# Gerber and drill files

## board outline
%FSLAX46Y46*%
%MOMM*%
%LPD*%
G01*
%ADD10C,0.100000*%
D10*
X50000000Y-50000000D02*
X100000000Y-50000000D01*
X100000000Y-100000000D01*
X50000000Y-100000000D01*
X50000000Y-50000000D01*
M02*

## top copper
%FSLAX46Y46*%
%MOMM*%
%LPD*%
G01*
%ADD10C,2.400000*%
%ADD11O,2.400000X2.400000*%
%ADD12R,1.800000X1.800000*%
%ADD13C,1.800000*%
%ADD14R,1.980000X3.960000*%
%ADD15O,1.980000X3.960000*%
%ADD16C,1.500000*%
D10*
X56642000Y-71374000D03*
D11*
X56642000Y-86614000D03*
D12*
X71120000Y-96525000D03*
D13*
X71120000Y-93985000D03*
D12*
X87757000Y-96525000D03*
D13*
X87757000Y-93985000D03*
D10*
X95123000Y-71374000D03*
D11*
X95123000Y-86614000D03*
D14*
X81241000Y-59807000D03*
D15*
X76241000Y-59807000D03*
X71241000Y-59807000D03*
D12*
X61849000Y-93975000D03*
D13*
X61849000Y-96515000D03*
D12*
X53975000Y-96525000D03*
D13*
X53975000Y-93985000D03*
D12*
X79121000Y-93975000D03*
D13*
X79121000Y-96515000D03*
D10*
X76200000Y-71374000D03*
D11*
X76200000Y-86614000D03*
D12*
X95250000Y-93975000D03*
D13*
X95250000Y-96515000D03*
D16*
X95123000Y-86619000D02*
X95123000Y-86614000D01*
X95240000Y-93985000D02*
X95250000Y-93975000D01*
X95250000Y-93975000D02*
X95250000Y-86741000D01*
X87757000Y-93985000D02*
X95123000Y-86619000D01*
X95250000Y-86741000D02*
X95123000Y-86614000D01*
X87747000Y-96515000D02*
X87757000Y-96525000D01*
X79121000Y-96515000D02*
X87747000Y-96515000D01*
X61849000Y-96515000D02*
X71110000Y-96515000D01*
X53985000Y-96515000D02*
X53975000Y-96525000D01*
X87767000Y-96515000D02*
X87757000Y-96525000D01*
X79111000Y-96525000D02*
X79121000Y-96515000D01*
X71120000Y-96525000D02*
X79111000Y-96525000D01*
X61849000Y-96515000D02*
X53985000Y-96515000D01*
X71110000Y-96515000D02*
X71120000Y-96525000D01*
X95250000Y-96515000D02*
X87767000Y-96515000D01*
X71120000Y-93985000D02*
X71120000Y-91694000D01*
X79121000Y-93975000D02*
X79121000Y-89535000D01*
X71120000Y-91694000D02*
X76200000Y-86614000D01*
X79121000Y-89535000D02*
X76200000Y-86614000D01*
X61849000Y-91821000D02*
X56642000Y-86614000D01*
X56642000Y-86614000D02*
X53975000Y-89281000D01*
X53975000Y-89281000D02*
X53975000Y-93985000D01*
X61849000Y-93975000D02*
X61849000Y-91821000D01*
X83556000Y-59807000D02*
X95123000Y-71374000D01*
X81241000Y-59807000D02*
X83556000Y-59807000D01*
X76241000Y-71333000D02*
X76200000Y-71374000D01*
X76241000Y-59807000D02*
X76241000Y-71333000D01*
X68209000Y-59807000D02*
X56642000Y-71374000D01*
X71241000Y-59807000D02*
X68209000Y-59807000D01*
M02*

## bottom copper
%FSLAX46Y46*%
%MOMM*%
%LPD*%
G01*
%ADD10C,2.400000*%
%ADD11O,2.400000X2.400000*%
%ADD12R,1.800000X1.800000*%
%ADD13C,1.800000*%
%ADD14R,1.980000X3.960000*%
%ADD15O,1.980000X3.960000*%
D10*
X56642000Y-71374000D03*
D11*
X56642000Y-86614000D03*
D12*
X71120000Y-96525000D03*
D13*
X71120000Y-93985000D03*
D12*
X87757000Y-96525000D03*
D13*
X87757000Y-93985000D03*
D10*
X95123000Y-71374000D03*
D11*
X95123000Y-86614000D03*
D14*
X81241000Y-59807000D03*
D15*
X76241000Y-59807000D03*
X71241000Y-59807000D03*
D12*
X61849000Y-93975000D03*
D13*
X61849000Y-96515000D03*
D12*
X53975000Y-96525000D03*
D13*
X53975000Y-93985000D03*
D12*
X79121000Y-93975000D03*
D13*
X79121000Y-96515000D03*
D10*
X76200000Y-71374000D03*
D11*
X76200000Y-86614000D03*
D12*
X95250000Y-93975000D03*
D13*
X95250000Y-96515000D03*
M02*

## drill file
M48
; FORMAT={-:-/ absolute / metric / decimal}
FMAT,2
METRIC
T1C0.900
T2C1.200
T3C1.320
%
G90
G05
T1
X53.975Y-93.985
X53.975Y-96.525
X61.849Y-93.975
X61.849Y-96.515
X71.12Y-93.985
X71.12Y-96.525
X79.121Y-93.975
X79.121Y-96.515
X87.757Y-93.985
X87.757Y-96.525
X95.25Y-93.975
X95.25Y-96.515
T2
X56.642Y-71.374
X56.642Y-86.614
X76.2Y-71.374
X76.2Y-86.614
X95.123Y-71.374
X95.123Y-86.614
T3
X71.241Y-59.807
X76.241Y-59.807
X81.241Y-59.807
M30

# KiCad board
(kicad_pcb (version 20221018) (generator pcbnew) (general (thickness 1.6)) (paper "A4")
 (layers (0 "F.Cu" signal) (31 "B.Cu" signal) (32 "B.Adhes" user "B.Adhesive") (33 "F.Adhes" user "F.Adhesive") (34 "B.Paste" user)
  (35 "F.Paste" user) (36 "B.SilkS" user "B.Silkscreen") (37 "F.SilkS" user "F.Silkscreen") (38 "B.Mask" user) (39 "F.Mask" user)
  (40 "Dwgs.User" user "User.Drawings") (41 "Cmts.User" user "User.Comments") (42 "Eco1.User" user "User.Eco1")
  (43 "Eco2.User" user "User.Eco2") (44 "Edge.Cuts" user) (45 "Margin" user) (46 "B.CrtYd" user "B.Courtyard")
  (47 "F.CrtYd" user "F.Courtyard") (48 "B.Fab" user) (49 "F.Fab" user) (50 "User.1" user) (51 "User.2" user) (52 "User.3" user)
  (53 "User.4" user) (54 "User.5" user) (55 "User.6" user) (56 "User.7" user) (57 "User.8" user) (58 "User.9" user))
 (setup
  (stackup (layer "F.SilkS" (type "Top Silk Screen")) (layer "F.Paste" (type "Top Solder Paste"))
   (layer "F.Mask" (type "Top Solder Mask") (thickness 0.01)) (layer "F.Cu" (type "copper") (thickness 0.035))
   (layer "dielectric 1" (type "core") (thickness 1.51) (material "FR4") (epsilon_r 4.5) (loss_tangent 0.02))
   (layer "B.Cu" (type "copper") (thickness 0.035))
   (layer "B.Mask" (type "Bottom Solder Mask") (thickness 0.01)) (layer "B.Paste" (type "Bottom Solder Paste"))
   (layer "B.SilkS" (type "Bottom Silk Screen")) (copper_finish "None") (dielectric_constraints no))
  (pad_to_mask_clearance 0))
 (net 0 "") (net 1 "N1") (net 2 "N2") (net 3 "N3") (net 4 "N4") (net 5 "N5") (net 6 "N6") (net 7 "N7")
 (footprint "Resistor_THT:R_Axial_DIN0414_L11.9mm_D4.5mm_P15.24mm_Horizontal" (layer "F.Cu") (at 56.642 71.374 -90)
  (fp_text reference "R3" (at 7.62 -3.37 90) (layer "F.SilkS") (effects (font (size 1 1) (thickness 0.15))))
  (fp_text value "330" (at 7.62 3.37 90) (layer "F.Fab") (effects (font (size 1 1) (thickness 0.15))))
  (pad "1" thru_hole circle (at 0 0 270) (size 2.4 2.4) (drill 1.2) (layers "*.Cu" "*.Mask") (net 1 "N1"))
  (pad "2" thru_hole oval (at 15.24 0 270) (size 2.4 2.4) (drill 1.2) (layers "*.Cu" "*.Mask") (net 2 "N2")))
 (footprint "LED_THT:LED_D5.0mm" (layer "F.Cu") (at 71.12 96.525 90)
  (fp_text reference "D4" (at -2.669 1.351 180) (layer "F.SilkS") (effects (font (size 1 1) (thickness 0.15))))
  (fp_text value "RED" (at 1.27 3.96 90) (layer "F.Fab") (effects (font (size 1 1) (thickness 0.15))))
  (pad "1" thru_hole rect (at 0 0 90) (size 1.8 1.8) (drill 0.9) (layers "*.Cu" "*.Mask") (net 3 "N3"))
  (pad "2" thru_hole circle (at 2.54 0 90) (size 1.8 1.8) (drill 0.9) (layers "*.Cu" "*.Mask") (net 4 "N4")))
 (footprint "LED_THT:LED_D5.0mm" (layer "F.Cu") (at 87.757 96.525 90)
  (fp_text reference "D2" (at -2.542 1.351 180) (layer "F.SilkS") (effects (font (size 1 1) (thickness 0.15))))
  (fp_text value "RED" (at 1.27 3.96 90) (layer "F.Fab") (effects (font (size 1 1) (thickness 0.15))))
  (pad "1" thru_hole rect (at 0 0 90) (size 1.8 1.8) (drill 0.9) (layers "*.Cu" "*.Mask") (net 3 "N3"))
  (pad "2" thru_hole circle (at 2.54 0 90) (size 1.8 1.8) (drill 0.9) (layers "*.Cu" "*.Mask") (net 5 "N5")))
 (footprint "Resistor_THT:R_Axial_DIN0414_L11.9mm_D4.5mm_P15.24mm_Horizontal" (layer "F.Cu") (at 95.123 71.374 -90)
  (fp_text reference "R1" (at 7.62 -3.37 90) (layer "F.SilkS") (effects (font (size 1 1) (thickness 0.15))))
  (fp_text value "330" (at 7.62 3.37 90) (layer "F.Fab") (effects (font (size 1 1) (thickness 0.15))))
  (pad "1" thru_hole circle (at 0 0 270) (size 2.4 2.4) (drill 1.2) (layers "*.Cu" "*.Mask") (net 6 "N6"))
  (pad "2" thru_hole oval (at 15.24 0 270) (size 2.4 2.4) (drill 1.2) (layers "*.Cu" "*.Mask") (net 5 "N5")))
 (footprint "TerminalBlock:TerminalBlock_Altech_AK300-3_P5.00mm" (layer "F.Cu") (at 81.241 59.807 180)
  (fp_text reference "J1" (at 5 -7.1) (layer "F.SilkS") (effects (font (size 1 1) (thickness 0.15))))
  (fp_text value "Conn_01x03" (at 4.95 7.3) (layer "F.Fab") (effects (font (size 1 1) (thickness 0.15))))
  (pad "1" thru_hole rect (at 0 0 180) (size 1.98 3.96) (drill 1.32) (layers "*.Cu" "*.Mask") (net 6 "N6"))
  (pad "2" thru_hole oval (at 5 0 180) (size 1.98 3.96) (drill 1.32) (layers "*.Cu" "*.Mask") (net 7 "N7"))
  (pad "3" thru_hole oval (at 10 0 180) (size 1.98 3.96) (drill 1.32) (layers "*.Cu" "*.Mask") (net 1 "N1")))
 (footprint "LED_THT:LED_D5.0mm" (layer "F.Cu") (at 61.849 93.975 -90)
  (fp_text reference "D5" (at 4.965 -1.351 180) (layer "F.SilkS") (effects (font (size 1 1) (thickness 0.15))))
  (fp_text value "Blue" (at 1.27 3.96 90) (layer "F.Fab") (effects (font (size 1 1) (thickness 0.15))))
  (pad "1" thru_hole rect (at 0 0 270) (size 1.8 1.8) (drill 0.9) (layers "*.Cu" "*.Mask") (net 2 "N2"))
  (pad "2" thru_hole circle (at 2.54 0 270) (size 1.8 1.8) (drill 0.9) (layers "*.Cu" "*.Mask") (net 3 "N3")))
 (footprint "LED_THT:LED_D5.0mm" (layer "F.Cu") (at 53.975 96.525 90)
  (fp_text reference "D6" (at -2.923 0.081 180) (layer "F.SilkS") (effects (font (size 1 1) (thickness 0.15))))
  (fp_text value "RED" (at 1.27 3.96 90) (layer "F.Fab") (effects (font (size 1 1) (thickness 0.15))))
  (pad "1" thru_hole rect (at 0 0 90) (size 1.8 1.8) (drill 0.9) (layers "*.Cu" "*.Mask") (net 3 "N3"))
  (pad "2" thru_hole circle (at 2.54 0 90) (size 1.8 1.8) (drill 0.9) (layers "*.Cu" "*.Mask") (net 2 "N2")))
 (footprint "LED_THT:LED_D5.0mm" (layer "F.Cu") (at 79.121 93.975 -90)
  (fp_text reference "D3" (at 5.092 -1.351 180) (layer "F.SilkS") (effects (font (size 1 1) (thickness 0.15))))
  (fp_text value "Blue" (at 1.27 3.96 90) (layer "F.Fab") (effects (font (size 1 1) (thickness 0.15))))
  (pad "1" thru_hole rect (at 0 0 270) (size 1.8 1.8) (drill 0.9) (layers "*.Cu" "*.Mask") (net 4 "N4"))
  (pad "2" thru_hole circle (at 2.54 0 270) (size 1.8 1.8) (drill 0.9) (layers "*.Cu" "*.Mask") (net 3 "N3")))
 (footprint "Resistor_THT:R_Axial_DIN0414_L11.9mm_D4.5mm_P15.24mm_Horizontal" (layer "F.Cu") (at 76.2 71.374 -90)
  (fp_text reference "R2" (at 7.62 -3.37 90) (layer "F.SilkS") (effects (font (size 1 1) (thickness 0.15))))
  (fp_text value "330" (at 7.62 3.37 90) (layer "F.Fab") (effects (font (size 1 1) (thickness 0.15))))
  (pad "1" thru_hole circle (at 0 0 270) (size 2.4 2.4) (drill 1.2) (layers "*.Cu" "*.Mask") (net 7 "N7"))
  (pad "2" thru_hole oval (at 15.24 0 270) (size 2.4 2.4) (drill 1.2) (layers "*.Cu" "*.Mask") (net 4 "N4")))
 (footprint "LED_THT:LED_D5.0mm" (layer "F.Cu") (at 95.25 93.975 -90)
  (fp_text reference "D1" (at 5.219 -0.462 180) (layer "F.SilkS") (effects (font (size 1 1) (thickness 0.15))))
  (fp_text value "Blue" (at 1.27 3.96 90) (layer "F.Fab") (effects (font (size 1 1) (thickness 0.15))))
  (pad "1" thru_hole rect (at 0 0 270) (size 1.8 1.8) (drill 0.9) (layers "*.Cu" "*.Mask") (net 5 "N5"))
  (pad "2" thru_hole circle (at 2.54 0 270) (size 1.8 1.8) (drill 0.9) (layers "*.Cu" "*.Mask") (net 3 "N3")))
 (gr_rect (start 50 50) (end 100 100) (stroke (width 0.1) (type solid)) (fill none) (layer "Edge.Cuts"))
 (segment (start 95.123 86.619) (end 95.123 86.614) (width 1.5) (layer "F.Cu") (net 5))
 (segment (start 95.24 93.985) (end 95.25 93.975) (width 1.5) (layer "F.Cu") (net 5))
 (segment (start 95.25 93.975) (end 95.25 86.741) (width 1.5) (layer "F.Cu") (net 5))
 (segment (start 87.757 93.985) (end 95.123 86.619) (width 1.5) (layer "F.Cu") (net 5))
 (segment (start 95.25 86.741) (end 95.123 86.614) (width 1.5) (layer "F.Cu") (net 5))
 (segment (start 87.747 96.515) (end 87.757 96.525) (width 1.5) (layer "F.Cu") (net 3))
 (segment (start 79.121 96.515) (end 87.747 96.515) (width 1.5) (layer "F.Cu") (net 3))
 (segment (start 61.849 96.515) (end 71.11 96.515) (width 1.5) (layer "F.Cu") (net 3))
 (segment (start 53.985 96.515) (end 53.975 96.525) (width 1.5) (layer "F.Cu") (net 3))
 (segment (start 87.767 96.515) (end 87.757 96.525) (width 1.5) (layer "F.Cu") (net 3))
 (segment (start 79.111 96.525) (end 79.121 96.515) (width 1.5) (layer "F.Cu") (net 3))
 (segment (start 71.12 96.525) (end 79.111 96.525) (width 1.5) (layer "F.Cu") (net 3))
 (segment (start 61.849 96.515) (end 53.985 96.515) (width 1.5) (layer "F.Cu") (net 3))
 (segment (start 71.11 96.515) (end 71.12 96.525) (width 1.5) (layer "F.Cu") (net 3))
 (segment (start 95.25 96.515) (end 87.767 96.515) (width 1.5) (layer "F.Cu") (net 3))
 (segment (start 71.12 93.985) (end 71.12 91.694) (width 1.5) (layer "F.Cu") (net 4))
 (segment (start 79.121 93.975) (end 79.121 89.535) (width 1.5) (layer "F.Cu") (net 4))
 (segment (start 71.12 91.694) (end 76.2 86.614) (width 1.5) (layer "F.Cu") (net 4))
 (segment (start 79.121 89.535) (end 76.2 86.614) (width 1.5) (layer "F.Cu") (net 4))
 (segment (start 61.849 91.821) (end 56.642 86.614) (width 1.5) (layer "F.Cu") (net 2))
 (segment (start 56.642 86.614) (end 53.975 89.281) (width 1.5) (layer "F.Cu") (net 2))
 (segment (start 53.975 89.281) (end 53.975 93.985) (width 1.5) (layer "F.Cu") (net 2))
 (segment (start 61.849 93.975) (end 61.849 91.821) (width 1.5) (layer "F.Cu") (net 2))
 (segment (start 83.556 59.807) (end 95.123 71.374) (width 1.5) (layer "F.Cu") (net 6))
 (segment (start 81.241 59.807) (end 83.556 59.807) (width 1.5) (layer "F.Cu") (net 6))
 (segment (start 76.241 71.333) (end 76.2 71.374) (width 1.5) (layer "F.Cu") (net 7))
 (segment (start 76.241 59.807) (end 76.241 71.333) (width 1.5) (layer "F.Cu") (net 7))
 (segment (start 68.209 59.807) (end 56.642 71.374) (width 1.5) (layer "F.Cu") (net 1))
 (segment (start 71.241 59.807) (end 68.209 59.807) (width 1.5) (layer "F.Cu") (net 1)))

